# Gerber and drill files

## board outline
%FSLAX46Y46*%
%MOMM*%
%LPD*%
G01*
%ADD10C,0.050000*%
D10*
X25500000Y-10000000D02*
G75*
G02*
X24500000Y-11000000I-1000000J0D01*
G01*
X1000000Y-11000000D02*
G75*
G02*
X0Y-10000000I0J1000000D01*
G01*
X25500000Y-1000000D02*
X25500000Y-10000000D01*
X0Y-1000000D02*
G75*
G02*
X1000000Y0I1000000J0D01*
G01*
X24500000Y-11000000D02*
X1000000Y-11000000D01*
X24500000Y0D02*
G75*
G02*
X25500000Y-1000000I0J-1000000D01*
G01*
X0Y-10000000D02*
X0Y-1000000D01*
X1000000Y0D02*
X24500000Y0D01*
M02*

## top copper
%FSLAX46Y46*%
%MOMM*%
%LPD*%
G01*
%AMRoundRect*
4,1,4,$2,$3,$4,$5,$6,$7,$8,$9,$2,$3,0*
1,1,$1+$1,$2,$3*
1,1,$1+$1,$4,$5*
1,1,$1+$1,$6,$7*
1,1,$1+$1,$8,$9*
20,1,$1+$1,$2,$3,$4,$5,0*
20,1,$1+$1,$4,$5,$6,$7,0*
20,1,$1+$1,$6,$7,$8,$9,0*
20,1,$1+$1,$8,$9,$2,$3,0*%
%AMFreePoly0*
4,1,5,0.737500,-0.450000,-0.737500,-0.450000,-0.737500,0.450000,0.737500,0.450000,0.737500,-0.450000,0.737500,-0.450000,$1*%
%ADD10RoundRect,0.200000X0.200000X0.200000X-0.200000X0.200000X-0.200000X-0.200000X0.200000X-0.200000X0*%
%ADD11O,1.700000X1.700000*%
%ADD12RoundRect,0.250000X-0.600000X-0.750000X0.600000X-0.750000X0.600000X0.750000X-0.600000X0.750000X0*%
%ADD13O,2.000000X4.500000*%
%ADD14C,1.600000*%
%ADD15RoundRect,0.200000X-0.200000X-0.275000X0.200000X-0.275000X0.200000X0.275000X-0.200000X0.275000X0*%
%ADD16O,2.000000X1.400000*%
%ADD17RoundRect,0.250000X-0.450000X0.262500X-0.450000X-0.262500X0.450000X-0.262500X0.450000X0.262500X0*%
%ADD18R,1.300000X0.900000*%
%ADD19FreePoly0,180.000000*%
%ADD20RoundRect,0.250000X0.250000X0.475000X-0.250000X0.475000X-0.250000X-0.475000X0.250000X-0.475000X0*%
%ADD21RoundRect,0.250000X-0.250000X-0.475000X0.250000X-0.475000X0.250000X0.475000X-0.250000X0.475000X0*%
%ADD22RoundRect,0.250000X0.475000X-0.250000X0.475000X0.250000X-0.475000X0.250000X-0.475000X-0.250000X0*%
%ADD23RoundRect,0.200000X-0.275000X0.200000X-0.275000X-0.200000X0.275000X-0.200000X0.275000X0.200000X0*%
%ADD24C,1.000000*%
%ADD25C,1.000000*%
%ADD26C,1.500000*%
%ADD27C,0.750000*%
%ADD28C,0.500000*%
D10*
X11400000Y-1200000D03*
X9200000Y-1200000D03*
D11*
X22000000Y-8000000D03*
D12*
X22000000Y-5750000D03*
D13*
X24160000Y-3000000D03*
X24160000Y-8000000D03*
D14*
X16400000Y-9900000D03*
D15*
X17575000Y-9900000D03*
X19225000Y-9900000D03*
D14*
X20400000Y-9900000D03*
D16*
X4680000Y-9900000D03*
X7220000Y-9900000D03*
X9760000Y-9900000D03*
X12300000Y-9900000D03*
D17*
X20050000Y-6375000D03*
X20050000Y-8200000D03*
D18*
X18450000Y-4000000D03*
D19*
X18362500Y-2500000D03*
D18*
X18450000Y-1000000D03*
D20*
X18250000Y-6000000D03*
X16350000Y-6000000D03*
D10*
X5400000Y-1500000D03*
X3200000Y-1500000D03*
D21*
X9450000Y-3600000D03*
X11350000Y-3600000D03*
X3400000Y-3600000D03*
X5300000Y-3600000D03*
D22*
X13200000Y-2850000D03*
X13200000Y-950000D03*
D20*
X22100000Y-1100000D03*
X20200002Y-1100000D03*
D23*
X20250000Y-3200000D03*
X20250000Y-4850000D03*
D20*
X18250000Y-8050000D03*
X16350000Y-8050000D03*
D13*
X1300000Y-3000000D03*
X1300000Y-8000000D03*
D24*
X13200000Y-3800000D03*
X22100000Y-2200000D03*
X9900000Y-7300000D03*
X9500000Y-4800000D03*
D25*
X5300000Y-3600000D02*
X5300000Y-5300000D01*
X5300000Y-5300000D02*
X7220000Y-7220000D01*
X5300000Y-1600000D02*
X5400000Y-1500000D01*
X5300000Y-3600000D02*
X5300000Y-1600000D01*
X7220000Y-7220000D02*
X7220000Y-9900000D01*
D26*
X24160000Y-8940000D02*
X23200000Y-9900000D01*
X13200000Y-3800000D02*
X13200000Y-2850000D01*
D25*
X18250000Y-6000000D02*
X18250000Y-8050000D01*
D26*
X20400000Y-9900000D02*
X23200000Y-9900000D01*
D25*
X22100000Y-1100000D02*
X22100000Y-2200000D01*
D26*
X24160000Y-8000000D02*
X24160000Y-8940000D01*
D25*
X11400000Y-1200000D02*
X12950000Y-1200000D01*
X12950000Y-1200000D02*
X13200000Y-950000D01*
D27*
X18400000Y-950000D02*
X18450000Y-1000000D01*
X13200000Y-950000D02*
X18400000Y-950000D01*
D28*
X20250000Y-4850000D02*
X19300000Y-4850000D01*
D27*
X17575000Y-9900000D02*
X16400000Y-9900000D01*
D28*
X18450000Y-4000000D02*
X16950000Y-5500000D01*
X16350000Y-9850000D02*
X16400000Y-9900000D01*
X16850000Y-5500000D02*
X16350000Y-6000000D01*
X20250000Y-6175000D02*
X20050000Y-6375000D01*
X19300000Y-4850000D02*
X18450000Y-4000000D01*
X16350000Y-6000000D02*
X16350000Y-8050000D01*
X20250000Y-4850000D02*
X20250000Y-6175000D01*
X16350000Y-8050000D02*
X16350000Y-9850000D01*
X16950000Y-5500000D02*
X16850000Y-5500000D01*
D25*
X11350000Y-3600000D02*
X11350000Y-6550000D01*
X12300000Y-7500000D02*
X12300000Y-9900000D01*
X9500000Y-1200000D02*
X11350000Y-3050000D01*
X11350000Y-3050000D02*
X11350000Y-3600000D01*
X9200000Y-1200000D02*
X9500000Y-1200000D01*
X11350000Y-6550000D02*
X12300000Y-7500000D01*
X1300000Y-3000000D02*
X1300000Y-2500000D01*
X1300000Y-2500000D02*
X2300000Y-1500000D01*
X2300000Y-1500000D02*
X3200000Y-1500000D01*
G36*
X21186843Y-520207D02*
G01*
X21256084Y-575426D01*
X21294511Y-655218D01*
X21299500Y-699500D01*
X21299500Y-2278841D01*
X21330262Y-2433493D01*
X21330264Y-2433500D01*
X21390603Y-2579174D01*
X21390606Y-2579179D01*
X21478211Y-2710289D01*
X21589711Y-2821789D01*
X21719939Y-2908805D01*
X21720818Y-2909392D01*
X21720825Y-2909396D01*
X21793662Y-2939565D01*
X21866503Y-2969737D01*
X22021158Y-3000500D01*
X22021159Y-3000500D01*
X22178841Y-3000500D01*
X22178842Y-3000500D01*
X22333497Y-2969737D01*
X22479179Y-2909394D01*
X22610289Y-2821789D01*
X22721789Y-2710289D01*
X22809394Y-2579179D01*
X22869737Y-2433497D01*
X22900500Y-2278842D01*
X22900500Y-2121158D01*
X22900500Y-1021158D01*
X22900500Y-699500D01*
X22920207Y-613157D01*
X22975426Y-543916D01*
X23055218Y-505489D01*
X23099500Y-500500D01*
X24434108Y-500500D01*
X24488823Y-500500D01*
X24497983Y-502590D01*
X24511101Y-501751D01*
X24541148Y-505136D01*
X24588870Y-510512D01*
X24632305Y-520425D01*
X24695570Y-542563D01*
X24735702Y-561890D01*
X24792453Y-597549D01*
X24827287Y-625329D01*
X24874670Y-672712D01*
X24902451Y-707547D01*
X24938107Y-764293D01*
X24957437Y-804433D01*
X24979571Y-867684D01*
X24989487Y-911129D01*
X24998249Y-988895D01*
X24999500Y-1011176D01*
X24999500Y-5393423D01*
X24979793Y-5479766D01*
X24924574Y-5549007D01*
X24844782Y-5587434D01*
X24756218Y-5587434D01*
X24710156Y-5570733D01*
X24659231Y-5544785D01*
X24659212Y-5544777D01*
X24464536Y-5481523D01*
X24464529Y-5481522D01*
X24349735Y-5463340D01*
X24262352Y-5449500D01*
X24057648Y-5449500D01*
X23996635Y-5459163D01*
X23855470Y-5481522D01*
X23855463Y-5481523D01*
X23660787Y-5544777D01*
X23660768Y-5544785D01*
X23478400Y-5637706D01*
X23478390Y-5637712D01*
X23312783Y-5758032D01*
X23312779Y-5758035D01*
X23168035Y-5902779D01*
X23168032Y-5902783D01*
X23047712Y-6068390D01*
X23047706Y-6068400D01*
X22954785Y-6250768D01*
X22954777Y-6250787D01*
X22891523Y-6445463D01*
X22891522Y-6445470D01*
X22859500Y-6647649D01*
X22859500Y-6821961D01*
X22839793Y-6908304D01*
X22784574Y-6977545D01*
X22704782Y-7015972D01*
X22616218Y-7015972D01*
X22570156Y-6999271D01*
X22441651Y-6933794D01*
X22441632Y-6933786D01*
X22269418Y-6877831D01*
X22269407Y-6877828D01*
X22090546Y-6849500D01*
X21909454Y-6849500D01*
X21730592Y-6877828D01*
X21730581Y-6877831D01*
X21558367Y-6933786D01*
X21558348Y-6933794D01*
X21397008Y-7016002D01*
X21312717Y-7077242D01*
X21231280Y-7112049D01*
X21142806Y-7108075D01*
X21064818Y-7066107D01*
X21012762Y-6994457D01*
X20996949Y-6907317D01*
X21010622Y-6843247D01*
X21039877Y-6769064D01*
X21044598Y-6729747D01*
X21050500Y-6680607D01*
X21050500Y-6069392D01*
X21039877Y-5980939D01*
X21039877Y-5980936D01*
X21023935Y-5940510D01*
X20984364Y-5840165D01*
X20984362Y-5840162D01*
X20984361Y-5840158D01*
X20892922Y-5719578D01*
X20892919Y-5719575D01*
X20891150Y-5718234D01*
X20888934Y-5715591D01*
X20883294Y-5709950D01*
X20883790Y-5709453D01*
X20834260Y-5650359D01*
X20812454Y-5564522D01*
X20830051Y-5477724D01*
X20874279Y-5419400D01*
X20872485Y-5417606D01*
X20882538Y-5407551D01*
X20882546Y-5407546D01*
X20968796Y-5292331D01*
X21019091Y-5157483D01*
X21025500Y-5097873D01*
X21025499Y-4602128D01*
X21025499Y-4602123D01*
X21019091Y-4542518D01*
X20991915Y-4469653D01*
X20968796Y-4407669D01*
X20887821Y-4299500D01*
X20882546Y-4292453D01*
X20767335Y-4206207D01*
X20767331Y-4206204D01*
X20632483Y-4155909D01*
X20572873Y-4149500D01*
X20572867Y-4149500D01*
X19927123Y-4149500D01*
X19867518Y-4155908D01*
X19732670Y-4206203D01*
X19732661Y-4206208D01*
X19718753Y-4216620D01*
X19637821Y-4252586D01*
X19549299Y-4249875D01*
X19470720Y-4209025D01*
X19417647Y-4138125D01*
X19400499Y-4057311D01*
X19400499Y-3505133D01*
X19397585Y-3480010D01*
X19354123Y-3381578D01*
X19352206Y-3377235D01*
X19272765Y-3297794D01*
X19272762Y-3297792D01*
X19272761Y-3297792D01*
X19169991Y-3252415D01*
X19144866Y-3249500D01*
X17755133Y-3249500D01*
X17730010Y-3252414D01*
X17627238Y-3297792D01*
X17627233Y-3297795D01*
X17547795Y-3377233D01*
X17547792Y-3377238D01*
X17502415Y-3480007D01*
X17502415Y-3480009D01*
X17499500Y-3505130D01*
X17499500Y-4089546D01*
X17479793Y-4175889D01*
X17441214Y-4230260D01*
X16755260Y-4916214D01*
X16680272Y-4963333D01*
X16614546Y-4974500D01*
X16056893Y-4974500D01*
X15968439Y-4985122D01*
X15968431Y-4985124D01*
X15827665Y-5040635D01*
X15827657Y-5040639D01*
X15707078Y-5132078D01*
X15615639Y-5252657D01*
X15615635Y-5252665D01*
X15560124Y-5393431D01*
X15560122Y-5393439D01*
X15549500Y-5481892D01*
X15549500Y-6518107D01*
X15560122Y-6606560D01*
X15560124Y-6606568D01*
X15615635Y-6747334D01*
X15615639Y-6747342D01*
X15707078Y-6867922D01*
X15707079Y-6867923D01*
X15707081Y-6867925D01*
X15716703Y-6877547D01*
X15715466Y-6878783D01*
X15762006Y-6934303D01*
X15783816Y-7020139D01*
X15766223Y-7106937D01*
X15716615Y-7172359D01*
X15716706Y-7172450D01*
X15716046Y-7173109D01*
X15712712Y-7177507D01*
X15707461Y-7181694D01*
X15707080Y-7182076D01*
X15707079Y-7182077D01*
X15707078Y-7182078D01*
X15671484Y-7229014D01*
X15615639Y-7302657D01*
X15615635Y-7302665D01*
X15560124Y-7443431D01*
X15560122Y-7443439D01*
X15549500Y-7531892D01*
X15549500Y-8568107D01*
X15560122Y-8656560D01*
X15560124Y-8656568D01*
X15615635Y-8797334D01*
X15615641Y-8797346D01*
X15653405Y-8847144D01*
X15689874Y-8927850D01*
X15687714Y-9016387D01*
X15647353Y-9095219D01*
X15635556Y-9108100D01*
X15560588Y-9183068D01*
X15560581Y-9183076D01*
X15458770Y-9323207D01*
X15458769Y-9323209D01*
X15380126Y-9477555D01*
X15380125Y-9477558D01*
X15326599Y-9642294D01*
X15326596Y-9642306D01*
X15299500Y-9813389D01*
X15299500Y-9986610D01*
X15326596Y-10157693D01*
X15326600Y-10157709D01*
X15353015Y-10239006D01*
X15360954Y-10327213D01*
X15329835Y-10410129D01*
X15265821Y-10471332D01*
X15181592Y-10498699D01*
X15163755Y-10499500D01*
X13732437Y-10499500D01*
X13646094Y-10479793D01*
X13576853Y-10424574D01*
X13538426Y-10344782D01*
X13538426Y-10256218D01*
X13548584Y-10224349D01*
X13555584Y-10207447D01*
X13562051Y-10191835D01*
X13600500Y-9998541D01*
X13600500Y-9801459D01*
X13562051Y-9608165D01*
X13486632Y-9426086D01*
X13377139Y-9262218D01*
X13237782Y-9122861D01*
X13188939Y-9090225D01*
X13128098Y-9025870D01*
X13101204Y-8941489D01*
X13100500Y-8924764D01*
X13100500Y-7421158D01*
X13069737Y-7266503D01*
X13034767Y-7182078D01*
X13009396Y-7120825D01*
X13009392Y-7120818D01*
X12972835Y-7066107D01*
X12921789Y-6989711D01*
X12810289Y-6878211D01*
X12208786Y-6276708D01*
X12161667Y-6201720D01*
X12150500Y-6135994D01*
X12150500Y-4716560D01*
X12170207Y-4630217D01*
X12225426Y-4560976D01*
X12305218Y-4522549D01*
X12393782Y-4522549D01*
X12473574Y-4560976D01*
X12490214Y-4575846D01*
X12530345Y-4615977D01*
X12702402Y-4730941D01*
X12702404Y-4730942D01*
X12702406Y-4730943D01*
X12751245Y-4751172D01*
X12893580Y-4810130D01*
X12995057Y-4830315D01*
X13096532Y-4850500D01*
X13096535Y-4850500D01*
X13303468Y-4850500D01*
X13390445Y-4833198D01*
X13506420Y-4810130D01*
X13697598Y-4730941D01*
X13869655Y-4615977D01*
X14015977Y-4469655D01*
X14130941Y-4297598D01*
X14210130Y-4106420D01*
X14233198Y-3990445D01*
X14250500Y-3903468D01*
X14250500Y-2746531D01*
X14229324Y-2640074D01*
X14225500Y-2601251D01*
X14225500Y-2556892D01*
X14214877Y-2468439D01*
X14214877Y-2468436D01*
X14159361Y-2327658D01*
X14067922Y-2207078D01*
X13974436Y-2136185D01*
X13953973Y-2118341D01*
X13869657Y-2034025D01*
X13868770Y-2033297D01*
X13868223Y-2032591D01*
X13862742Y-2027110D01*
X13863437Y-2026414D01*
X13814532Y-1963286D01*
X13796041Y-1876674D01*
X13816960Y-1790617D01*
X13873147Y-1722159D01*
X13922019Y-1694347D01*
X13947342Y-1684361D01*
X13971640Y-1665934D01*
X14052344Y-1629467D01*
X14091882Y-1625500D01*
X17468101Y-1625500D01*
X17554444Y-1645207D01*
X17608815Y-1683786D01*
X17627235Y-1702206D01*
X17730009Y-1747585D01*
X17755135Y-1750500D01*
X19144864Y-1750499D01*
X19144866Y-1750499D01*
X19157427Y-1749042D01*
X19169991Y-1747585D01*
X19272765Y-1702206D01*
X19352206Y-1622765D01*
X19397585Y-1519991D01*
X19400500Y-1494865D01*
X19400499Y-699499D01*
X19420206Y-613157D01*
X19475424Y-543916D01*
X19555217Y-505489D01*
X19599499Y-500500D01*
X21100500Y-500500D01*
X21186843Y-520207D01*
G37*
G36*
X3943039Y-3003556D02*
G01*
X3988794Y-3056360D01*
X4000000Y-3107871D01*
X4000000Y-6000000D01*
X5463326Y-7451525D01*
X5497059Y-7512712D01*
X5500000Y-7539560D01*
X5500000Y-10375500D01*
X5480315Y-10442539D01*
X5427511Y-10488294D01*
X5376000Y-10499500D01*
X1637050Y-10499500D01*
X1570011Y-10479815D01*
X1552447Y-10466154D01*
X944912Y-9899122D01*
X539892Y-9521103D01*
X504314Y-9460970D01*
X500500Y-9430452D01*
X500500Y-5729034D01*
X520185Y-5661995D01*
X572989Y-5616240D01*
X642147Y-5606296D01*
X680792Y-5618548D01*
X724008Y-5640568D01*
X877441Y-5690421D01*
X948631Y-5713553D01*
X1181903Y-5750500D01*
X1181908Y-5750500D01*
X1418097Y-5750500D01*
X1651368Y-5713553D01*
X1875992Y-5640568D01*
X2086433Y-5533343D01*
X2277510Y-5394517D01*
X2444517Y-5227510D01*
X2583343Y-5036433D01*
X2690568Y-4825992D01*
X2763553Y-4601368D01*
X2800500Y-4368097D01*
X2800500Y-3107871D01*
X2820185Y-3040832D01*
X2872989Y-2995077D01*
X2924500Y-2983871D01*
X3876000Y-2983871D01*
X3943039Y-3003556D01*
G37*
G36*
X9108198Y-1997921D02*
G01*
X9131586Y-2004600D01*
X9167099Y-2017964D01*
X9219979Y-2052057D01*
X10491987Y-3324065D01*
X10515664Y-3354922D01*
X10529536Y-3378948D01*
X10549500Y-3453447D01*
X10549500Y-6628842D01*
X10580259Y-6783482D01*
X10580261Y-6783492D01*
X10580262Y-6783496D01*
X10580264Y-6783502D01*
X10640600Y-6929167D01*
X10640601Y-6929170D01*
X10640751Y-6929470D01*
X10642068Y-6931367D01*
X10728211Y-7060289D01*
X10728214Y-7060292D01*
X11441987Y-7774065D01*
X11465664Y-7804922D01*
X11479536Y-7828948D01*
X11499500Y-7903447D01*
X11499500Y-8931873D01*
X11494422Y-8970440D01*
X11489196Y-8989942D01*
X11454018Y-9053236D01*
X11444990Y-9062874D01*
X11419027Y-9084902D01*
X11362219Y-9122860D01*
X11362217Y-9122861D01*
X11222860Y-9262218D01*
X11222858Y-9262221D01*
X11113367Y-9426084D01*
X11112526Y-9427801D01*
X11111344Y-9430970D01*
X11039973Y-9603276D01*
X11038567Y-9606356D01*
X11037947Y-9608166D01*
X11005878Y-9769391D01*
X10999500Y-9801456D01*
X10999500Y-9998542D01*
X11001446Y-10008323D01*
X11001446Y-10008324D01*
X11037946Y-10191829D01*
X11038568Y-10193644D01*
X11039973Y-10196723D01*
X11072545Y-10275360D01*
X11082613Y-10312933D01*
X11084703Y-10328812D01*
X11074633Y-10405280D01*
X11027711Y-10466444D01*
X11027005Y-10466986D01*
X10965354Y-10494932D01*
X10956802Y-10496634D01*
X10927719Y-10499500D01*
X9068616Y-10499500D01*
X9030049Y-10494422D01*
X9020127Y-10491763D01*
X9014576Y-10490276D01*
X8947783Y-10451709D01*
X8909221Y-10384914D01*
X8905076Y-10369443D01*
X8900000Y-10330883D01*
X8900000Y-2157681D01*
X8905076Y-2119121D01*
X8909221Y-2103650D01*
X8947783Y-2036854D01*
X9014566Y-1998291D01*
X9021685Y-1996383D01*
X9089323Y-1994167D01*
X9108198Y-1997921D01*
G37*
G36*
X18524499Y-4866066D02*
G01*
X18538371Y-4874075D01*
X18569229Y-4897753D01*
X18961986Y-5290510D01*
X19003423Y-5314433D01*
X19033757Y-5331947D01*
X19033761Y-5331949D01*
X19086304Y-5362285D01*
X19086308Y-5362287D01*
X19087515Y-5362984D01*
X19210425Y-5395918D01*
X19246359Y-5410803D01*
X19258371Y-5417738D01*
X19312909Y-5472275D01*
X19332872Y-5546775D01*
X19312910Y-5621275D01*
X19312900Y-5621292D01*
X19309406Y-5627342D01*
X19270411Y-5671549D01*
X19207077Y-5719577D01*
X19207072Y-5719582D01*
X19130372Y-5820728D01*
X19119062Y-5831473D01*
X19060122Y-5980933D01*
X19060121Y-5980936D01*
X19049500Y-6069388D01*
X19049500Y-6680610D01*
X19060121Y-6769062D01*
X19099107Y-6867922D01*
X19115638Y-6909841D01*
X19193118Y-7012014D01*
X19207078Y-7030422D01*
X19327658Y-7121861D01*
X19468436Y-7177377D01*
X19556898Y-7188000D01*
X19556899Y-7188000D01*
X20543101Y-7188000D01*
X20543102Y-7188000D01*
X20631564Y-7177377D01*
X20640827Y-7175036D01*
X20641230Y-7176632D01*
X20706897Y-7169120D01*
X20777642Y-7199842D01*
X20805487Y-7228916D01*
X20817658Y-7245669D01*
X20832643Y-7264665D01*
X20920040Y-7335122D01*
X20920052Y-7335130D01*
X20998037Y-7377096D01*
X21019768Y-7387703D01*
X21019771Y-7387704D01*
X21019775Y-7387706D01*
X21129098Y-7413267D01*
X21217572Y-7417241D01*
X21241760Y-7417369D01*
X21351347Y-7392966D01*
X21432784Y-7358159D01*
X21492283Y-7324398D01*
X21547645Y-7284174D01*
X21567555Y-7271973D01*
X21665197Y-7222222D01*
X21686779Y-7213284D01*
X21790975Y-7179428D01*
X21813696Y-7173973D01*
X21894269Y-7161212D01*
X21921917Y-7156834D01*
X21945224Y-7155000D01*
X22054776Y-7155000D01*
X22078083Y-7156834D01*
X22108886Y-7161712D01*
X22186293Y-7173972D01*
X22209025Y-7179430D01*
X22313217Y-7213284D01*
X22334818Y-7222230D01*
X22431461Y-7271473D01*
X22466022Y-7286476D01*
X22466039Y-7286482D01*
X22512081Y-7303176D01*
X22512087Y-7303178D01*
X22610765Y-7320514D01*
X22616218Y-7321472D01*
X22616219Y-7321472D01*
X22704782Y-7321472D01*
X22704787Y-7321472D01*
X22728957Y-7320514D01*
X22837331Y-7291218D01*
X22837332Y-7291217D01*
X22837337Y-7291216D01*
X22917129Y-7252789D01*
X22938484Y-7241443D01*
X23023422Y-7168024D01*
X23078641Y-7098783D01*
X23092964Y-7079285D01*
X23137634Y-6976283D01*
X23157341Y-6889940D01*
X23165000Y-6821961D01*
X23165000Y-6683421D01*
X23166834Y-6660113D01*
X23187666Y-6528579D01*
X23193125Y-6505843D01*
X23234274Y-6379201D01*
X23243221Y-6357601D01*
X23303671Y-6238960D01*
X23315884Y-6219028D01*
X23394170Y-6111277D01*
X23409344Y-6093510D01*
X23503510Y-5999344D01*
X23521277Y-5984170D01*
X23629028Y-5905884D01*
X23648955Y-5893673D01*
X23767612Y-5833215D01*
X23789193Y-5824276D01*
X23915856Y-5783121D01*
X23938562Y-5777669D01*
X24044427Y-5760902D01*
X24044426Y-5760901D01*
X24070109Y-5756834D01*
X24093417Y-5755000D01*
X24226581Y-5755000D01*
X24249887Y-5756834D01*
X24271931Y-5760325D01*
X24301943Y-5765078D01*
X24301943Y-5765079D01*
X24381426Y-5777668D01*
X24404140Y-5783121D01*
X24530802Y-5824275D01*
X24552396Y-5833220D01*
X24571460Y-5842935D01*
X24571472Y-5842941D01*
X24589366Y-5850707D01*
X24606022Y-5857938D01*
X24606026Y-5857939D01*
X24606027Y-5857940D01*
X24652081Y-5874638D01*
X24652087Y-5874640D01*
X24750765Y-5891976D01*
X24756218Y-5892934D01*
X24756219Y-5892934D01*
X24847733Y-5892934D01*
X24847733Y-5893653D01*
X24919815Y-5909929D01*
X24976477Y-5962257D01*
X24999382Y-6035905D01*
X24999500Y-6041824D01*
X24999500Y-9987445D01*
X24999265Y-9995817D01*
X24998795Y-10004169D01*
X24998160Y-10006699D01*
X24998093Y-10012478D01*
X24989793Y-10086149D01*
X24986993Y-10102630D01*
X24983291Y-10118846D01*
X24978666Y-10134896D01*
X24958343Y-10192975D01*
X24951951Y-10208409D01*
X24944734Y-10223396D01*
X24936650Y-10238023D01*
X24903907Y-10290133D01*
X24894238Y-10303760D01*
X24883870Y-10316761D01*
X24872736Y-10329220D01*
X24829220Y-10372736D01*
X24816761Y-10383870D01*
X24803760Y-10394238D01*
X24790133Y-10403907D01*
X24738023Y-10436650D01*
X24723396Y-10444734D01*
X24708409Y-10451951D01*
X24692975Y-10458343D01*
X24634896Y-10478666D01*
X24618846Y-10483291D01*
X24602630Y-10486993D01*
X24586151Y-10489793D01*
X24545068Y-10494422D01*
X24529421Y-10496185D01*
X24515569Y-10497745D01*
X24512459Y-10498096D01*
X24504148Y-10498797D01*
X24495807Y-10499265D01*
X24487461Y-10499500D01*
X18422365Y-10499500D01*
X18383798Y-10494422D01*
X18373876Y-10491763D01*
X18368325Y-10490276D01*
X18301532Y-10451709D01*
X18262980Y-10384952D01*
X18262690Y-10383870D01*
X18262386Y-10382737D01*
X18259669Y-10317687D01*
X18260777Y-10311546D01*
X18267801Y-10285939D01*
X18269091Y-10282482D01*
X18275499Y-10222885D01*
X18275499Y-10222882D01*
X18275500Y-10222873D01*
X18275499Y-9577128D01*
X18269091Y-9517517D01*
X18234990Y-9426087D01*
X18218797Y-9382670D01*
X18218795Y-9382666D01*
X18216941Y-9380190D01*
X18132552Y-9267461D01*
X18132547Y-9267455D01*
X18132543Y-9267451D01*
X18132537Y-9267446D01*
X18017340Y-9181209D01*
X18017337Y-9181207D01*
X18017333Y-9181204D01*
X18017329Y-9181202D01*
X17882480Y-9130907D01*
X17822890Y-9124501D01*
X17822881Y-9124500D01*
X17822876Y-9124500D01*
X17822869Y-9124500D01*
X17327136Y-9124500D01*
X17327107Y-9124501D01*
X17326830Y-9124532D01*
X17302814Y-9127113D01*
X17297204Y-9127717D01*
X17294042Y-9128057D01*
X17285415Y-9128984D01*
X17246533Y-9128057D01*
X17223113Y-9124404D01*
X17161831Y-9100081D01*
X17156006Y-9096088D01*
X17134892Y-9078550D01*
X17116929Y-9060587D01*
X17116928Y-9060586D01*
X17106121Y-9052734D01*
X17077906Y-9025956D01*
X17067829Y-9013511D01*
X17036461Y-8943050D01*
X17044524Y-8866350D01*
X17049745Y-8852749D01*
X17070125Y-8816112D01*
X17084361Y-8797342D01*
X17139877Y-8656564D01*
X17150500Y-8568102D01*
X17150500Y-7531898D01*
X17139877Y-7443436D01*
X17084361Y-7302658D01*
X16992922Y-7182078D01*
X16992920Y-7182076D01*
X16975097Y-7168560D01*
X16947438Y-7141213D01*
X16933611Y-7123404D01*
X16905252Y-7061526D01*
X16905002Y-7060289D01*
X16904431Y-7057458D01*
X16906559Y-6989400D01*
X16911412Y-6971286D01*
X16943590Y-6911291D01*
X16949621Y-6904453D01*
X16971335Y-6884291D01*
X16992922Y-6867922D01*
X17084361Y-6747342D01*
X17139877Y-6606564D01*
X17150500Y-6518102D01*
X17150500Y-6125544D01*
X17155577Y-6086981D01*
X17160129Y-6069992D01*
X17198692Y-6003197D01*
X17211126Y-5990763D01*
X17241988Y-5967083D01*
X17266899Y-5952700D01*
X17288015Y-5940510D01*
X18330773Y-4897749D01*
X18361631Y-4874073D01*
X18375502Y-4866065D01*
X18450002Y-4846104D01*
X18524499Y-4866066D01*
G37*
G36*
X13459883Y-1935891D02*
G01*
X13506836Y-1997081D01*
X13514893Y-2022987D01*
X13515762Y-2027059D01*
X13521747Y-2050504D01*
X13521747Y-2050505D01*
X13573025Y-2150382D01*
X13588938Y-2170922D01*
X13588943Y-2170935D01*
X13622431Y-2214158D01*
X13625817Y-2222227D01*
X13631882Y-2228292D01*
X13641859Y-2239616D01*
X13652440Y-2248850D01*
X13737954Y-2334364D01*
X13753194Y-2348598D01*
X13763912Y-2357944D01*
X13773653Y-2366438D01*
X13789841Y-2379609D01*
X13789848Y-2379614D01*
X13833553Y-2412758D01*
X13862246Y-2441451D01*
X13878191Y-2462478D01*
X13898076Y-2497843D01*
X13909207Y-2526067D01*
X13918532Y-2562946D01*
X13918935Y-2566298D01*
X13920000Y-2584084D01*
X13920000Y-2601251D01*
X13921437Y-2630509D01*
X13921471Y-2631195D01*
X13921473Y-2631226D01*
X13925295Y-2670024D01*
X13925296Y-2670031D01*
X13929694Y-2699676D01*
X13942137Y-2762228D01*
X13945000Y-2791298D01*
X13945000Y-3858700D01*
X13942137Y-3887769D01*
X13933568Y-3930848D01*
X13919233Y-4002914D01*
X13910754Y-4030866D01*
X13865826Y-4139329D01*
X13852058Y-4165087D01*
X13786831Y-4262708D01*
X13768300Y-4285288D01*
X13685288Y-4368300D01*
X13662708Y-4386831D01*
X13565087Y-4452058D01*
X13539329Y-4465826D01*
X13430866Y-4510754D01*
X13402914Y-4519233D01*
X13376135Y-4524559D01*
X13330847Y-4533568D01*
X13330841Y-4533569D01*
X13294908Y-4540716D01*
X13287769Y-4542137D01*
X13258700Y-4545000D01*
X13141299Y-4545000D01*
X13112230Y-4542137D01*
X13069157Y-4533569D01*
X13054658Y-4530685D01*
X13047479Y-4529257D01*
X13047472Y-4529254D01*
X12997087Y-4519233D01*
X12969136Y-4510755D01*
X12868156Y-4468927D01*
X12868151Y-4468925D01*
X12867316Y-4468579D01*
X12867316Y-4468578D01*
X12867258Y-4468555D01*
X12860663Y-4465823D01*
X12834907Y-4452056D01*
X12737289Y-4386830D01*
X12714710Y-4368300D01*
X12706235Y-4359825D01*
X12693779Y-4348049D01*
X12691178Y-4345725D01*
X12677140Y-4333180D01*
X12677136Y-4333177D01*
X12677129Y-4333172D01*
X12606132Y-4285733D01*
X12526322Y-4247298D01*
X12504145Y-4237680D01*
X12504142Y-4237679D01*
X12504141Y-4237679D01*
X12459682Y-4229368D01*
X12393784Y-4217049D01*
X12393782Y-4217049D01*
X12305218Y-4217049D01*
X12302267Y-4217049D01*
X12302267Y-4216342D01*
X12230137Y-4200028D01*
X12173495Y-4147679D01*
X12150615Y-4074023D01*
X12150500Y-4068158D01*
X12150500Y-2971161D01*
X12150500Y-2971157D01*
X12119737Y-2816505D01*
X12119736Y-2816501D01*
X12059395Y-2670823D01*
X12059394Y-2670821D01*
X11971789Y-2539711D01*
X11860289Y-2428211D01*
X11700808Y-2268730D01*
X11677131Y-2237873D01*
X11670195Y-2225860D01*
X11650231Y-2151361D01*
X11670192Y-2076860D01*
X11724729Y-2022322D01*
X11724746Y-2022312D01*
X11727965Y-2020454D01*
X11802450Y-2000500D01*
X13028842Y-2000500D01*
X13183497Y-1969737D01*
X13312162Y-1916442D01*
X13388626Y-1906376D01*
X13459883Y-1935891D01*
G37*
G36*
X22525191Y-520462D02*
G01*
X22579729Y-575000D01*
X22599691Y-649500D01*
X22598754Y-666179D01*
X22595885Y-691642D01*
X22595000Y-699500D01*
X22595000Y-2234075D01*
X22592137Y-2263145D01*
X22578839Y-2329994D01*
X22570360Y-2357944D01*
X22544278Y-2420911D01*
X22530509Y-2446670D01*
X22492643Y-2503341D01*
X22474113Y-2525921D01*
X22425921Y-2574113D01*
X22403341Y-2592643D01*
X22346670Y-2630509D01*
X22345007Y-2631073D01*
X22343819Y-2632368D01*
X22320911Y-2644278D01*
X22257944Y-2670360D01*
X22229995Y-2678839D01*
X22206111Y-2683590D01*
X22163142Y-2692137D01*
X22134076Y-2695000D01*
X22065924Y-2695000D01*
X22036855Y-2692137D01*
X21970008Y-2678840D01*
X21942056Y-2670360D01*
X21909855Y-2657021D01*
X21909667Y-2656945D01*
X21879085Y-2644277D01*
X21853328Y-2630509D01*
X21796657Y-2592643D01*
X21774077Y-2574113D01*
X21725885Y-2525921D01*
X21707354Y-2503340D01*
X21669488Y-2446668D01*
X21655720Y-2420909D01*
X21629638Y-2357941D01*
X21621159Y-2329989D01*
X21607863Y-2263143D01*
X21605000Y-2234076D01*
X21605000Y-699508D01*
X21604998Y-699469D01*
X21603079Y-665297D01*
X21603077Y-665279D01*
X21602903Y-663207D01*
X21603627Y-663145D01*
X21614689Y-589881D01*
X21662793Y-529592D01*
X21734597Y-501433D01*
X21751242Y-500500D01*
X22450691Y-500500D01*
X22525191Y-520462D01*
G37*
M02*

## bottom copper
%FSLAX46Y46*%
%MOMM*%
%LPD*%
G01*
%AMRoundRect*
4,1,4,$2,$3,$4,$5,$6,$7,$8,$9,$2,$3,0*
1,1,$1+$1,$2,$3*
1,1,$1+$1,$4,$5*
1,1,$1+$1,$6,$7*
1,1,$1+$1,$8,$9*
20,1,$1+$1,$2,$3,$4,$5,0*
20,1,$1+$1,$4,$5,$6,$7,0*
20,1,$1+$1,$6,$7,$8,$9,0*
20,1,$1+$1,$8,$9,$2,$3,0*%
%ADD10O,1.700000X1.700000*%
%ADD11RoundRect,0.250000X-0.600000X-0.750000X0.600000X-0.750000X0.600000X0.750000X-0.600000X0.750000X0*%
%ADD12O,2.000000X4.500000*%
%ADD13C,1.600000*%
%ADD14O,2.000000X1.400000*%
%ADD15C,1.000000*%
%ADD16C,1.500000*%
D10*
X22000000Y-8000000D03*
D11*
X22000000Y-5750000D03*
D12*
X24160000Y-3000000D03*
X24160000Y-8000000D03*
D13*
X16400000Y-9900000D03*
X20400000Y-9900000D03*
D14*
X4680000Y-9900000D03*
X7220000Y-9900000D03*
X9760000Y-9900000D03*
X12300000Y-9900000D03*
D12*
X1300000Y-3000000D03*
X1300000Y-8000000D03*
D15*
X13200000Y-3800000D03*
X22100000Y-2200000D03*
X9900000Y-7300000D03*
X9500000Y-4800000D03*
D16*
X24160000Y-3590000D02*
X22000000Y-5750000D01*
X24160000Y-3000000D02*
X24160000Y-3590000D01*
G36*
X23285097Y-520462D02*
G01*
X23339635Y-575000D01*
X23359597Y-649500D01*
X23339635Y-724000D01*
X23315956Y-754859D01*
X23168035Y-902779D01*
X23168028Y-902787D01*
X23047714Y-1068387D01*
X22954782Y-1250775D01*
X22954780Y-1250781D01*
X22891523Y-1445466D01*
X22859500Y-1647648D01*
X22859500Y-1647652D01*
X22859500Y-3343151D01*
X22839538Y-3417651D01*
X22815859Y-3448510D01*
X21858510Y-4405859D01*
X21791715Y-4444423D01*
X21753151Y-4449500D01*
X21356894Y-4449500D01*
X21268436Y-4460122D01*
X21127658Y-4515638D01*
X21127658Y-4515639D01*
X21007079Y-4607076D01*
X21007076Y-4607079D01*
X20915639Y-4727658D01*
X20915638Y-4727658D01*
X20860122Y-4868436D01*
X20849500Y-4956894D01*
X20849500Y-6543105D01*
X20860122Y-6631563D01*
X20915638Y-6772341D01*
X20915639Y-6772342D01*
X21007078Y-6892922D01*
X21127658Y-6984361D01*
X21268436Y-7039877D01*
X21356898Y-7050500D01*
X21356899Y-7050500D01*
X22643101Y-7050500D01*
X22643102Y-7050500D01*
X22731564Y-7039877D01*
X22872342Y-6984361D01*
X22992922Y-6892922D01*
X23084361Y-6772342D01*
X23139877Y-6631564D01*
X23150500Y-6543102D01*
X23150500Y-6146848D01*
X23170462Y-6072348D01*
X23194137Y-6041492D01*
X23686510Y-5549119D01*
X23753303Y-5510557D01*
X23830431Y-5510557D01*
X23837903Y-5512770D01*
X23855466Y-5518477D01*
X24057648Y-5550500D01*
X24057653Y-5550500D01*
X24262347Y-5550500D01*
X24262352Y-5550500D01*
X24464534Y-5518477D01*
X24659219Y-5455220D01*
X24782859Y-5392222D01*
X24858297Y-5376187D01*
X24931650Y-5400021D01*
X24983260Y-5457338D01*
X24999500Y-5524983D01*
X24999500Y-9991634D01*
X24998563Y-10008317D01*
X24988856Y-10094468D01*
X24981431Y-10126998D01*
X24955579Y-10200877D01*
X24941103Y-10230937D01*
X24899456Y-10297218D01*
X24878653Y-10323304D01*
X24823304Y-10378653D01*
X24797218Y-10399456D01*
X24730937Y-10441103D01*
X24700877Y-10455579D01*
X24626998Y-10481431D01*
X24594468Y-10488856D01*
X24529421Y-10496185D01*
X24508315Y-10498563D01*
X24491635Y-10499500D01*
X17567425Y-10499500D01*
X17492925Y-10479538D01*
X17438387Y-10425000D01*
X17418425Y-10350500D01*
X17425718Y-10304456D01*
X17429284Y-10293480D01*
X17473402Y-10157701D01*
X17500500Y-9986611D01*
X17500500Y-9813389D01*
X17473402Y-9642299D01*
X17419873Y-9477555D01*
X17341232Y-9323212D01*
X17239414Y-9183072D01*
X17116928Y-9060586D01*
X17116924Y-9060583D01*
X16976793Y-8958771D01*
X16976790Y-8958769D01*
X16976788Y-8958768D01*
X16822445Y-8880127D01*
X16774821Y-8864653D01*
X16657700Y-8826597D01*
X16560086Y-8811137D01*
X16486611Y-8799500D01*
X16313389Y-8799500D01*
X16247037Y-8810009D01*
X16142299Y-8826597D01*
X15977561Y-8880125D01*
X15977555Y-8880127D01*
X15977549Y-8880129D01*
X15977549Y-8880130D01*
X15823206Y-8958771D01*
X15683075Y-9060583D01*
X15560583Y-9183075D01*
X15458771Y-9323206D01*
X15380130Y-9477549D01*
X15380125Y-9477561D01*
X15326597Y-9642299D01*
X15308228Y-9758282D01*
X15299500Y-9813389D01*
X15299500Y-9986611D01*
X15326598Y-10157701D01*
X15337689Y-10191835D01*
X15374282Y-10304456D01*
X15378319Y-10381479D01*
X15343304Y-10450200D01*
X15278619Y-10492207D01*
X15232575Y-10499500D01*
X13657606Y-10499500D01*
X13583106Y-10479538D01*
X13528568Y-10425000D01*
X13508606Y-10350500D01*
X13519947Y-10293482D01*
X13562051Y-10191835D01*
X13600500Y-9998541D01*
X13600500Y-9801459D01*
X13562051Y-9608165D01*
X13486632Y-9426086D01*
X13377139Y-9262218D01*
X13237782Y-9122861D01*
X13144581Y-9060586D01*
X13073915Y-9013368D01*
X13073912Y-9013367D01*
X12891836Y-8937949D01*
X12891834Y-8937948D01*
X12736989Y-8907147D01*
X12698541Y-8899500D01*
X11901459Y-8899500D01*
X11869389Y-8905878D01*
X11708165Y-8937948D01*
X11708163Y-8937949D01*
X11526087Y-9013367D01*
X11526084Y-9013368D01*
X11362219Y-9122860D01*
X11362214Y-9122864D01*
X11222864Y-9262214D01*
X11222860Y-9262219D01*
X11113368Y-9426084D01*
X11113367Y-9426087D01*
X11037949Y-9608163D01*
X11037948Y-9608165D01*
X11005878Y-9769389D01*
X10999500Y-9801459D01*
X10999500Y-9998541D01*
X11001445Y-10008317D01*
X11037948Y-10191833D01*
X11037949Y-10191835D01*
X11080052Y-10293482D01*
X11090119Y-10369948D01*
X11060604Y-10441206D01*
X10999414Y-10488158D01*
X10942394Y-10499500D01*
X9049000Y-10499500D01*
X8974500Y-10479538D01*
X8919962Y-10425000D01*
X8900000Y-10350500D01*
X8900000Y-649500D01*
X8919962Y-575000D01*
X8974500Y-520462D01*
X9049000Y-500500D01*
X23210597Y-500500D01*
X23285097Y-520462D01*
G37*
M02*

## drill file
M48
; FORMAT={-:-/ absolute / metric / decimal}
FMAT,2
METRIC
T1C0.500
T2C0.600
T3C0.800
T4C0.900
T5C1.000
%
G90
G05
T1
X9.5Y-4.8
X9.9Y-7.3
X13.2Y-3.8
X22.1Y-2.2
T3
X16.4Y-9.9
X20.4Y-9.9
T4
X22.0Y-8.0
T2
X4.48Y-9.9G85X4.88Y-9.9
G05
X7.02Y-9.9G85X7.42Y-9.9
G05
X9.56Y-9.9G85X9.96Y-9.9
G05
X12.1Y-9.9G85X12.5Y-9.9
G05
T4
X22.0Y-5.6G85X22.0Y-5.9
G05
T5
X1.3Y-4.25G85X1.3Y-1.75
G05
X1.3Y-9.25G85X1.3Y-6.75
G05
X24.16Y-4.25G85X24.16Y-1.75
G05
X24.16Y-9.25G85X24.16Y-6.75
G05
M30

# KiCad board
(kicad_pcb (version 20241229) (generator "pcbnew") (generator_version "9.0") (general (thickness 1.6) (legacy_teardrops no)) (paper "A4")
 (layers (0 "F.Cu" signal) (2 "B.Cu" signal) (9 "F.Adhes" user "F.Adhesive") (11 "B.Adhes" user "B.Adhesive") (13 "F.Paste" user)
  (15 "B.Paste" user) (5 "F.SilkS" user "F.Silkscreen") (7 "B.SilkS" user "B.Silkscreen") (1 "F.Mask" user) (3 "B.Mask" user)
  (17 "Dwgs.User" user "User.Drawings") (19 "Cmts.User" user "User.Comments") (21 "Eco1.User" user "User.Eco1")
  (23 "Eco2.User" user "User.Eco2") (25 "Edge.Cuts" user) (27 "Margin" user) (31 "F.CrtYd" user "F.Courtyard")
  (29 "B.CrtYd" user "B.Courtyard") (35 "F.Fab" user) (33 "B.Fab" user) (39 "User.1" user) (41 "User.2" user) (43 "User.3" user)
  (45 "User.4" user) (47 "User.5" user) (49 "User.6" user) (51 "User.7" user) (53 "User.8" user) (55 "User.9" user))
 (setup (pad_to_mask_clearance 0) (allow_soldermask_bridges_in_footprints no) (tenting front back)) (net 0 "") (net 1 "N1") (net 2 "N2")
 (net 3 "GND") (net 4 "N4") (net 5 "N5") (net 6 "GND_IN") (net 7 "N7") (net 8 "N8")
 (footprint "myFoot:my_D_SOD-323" (layer "F.Cu") (at 10.3 1.2 180)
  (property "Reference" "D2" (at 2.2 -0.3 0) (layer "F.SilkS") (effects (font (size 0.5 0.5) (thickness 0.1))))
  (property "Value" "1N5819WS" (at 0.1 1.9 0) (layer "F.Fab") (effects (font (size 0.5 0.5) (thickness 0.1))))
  (pad "1" smd roundrect (at -1.1 0 180) (size 0.8 0.8) (layers "F.Cu" "F.Mask" "F.Paste") (roundrect_rratio 0.25) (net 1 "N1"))
  (pad "2" smd roundrect (at 1.1 0 180) (size 0.8 0.8) (layers "F.Cu" "F.Mask" "F.Paste") (roundrect_rratio 0.25) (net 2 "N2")))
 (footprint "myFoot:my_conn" (layer "F.Cu") (at 22 6.95)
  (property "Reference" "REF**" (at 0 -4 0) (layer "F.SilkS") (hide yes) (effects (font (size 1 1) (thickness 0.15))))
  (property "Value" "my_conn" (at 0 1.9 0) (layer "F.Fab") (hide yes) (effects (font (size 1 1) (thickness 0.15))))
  (pad "1" thru_hole oval (at 0 1.05) (size 1.7 1.7) (drill oval 0.9) (layers "*.Cu" "*.Mask") (remove_unused_layers no) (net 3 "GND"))
  (pad "2" thru_hole roundrect (at 0 -1.2) (size 1.7 2) (drill oval 0.9 1.2) (layers "*.Cu" "*.Mask") (remove_unused_layers no)
   (roundrect_rratio 0.1470588235) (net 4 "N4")))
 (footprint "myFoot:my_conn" (layer "F.Cu") (at 24.16 5.5 180)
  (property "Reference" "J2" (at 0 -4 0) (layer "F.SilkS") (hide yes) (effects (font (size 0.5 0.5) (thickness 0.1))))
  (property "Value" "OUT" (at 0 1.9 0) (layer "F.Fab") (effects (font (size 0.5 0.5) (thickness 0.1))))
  (pad "1" thru_hole oval (at 0 2.5 180) (size 2 4.5) (drill oval 1 3.5) (layers "*.Cu" "*.Mask") (remove_unused_layers no) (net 4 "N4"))
  (pad "2" thru_hole oval (at 0 -2.5 180) (size 2 4.5) (drill oval 1 3.5) (layers "*.Cu" "*.Mask") (remove_unused_layers no) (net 3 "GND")))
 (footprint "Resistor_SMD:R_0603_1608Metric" (layer "F.Cu") (at 18.4 9.9)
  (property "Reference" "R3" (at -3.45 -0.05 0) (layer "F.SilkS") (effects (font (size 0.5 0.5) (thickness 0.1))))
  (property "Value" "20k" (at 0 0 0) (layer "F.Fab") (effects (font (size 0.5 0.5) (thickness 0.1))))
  (pad "1" thru_hole circle (at -2 0) (size 1.6 1.6) (drill 0.8) (layers "*.Cu" "*.Mask") (remove_unused_layers no) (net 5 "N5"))
  (pad "1" smd roundrect (at -0.825 0) (size 0.8 0.95) (layers "F.Cu" "F.Mask" "F.Paste") (roundrect_rratio 0.25) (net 5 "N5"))
  (pad "2" smd roundrect (at 0.825 0) (size 0.8 0.95) (layers "F.Cu" "F.Mask" "F.Paste") (roundrect_rratio 0.25) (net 3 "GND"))
  (pad "2" thru_hole circle (at 2 0) (size 1.6 1.6) (drill 0.8) (layers "*.Cu" "*.Mask") (remove_unused_layers no) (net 3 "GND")))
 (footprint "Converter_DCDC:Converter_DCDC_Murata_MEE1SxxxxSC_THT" (layer "F.Cu") (at 8.49 9.9 90)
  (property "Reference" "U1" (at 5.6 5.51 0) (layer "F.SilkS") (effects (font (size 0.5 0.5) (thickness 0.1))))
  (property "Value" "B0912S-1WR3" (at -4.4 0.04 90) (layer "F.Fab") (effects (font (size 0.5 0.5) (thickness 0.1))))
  (pad "1" thru_hole oval (at 0 -3.81 90) (size 1.4 2) (drill oval 0.6 1) (layers "*.Cu" "*.Mask") (remove_unused_layers no)
   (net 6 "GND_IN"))
  (pad "2" thru_hole oval (at 0 -1.27 90) (size 1.4 2) (drill oval 0.6 1) (layers "*.Cu" "*.Mask") (remove_unused_layers no) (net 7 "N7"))
  (pad "3" thru_hole oval (at 0 1.27 90) (size 1.4 2) (drill oval 0.6 1) (layers "*.Cu" "*.Mask") (remove_unused_layers no) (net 3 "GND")
   (zone_connect 2))
  (pad "4" thru_hole oval (at 0 3.81 90) (size 1.4 2) (drill oval 0.6 1) (layers "*.Cu" "*.Mask") (remove_unused_layers no) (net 2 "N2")))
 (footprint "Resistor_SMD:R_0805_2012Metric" (layer "F.Cu") (at 20.05 7.2875 -90)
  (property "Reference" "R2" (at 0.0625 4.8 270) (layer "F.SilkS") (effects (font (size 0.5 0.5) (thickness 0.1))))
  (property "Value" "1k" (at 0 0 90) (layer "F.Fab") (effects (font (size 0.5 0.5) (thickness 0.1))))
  (pad "1" smd roundrect (at -0.9125 0 270) (size 1.025 1.4) (layers "F.Cu" "F.Mask" "F.Paste") (roundrect_rratio 0.243902) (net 5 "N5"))
  (pad "2" smd roundrect (at 0.9125 0 270) (size 1.025 1.4) (layers "F.Cu" "F.Mask" "F.Paste") (roundrect_rratio 0.243902) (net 3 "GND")))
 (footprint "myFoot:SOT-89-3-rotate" (layer "F.Cu") (at 17 2.5 180)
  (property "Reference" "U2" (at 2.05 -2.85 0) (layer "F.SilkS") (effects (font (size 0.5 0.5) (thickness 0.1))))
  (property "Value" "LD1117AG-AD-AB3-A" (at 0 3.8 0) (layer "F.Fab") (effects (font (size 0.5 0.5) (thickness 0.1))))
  (pad "1" smd rect (at -1.45 -1.5 180) (size 1.3 0.9) (layers "F.Cu" "F.Mask" "F.Paste") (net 5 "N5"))
  (pad "2" smd custom (at -1.3625 0 180) (size 1.475 0.9) (layers "F.Cu" "F.Mask" "F.Paste") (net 4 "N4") (zone_connect 2)
   (options (clearance outline) (anchor rect)) (primitives))
  (pad "3" smd rect (at -1.45 1.5 180) (size 1.3 0.9) (layers "F.Cu" "F.Mask" "F.Paste") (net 1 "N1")))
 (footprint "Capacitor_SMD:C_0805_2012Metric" (layer "F.Cu") (at 17.3 6 180)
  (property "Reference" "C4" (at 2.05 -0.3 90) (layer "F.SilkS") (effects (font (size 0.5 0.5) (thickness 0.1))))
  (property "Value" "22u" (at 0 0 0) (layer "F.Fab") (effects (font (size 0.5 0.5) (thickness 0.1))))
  (pad "1" smd roundrect (at -0.95 0 180) (size 1 1.45) (layers "F.Cu" "F.Mask" "F.Paste") (roundrect_rratio 0.25) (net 3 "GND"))
  (pad "2" smd roundrect (at 0.95 0 180) (size 1 1.45) (layers "F.Cu" "F.Mask" "F.Paste") (roundrect_rratio 0.25) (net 5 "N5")))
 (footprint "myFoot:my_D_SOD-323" (layer "F.Cu") (at 4.3 1.5 180)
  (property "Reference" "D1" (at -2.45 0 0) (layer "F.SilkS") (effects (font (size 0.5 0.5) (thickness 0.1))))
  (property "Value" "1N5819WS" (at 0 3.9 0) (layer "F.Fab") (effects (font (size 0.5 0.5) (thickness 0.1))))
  (pad "1" smd roundrect (at -1.1 0 180) (size 0.8 0.8) (layers "F.Cu" "F.Mask" "F.Paste") (roundrect_rratio 0.25) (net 7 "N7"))
  (pad "2" smd roundrect (at 1.1 0 180) (size 0.8 0.8) (layers "F.Cu" "F.Mask" "F.Paste") (roundrect_rratio 0.25) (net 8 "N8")))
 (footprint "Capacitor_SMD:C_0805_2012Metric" (layer "F.Cu") (at 10.4 3.6)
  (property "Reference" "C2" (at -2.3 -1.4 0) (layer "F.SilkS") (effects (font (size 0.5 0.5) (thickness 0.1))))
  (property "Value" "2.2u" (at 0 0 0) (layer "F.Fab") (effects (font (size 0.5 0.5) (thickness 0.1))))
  (pad "1" smd roundrect (at -0.95 0) (size 1 1.45) (layers "F.Cu" "F.Mask" "F.Paste") (roundrect_rratio 0.25) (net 3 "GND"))
  (pad "2" smd roundrect (at 0.95 0) (size 1 1.45) (layers "F.Cu" "F.Mask" "F.Paste") (roundrect_rratio 0.25) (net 2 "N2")))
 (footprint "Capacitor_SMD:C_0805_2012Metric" (layer "F.Cu") (at 4.35 3.6)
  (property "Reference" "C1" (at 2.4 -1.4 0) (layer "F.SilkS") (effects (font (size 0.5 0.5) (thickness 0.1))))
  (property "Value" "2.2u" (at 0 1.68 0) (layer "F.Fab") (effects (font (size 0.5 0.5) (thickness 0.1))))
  (pad "1" smd roundrect (at -0.95 0) (size 1 1.45) (layers "F.Cu" "F.Mask" "F.Paste") (roundrect_rratio 0.25) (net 6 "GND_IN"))
  (pad "2" smd roundrect (at 0.95 0) (size 1 1.45) (layers "F.Cu" "F.Mask" "F.Paste") (roundrect_rratio 0.25) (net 7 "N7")))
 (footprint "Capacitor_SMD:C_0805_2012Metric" (layer "F.Cu") (at 13.2 1.9 90)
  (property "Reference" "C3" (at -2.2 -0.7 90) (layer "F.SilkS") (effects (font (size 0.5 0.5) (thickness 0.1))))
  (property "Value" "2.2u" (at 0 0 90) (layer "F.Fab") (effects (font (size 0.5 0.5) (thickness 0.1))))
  (pad "1" smd roundrect (at -0.95 0 90) (size 1 1.45) (layers "F.Cu" "F.Mask" "F.Paste") (roundrect_rratio 0.25) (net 3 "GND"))
  (pad "2" smd roundrect (at 0.95 0 90) (size 1 1.45) (layers "F.Cu" "F.Mask" "F.Paste") (roundrect_rratio 0.25) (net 1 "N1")))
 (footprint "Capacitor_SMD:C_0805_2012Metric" (layer "F.Cu") (at 21.150001 1.1 180)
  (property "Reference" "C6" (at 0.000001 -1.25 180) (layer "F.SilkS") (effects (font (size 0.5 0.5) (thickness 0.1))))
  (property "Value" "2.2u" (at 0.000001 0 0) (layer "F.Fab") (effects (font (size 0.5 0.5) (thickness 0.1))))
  (pad "1" smd roundrect (at -0.949999 0 180) (size 1 1.45) (layers "F.Cu" "F.Mask" "F.Paste") (roundrect_rratio 0.25) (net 3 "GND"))
  (pad "2" smd roundrect (at 0.949999 0 180) (size 1 1.45) (layers "F.Cu" "F.Mask" "F.Paste") (roundrect_rratio 0.25) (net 4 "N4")))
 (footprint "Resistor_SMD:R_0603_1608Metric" (layer "F.Cu") (at 20.25 4.025 -90)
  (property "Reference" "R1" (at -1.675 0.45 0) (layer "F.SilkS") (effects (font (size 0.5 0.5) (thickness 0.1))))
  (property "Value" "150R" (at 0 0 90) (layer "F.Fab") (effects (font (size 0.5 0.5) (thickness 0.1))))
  (pad "1" smd roundrect (at -0.825 0 270) (size 0.8 0.95) (layers "F.Cu" "F.Mask" "F.Paste") (roundrect_rratio 0.25) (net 4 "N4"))
  (pad "2" smd roundrect (at 0.825 0 270) (size 0.8 0.95) (layers "F.Cu" "F.Mask" "F.Paste") (roundrect_rratio 0.25) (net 5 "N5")))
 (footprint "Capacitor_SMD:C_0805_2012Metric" (layer "F.Cu") (at 17.3 8.05 180)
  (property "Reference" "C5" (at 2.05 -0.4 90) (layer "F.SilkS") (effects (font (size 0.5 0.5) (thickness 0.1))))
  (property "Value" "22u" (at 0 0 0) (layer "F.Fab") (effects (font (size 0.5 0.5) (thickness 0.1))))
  (pad "1" smd roundrect (at -0.95 0 180) (size 1 1.45) (layers "F.Cu" "F.Mask" "F.Paste") (roundrect_rratio 0.25) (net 3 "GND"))
  (pad "2" smd roundrect (at 0.95 0 180) (size 1 1.45) (layers "F.Cu" "F.Mask" "F.Paste") (roundrect_rratio 0.25) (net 5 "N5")))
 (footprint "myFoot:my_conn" (layer "F.Cu") (at 1.3 5.5 180)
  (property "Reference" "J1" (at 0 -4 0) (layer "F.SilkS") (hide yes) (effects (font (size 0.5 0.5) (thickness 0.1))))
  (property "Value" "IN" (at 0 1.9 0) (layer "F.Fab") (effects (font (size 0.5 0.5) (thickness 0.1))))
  (pad "1" thru_hole oval (at 0 2.5 180) (size 2 4.5) (drill oval 1 3.5) (layers "*.Cu" "*.Mask") (remove_unused_layers no) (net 8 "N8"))
  (pad "2" thru_hole oval (at 0 -2.5 180) (size 2 4.5) (drill oval 1 3.5) (layers "*.Cu" "*.Mask") (remove_unused_layers no)
   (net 6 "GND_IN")))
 (gr_arc (start 25.5 10) (mid 25.207107 10.707107) (end 24.5 11) (stroke (width 0.05) (type default)) (layer "Edge.Cuts"))
 (gr_arc (start 1 11) (mid 0.292893 10.707107) (end 0 10) (stroke (width 0.05) (type default)) (layer "Edge.Cuts"))
 (gr_line (start 25.5 1) (end 25.5 10) (stroke (width 0.05) (type default)) (layer "Edge.Cuts"))
 (gr_arc (start 0 1) (mid 0.292893 0.292893) (end 1 0) (stroke (width 0.05) (type default)) (layer "Edge.Cuts"))
 (gr_line (start 24.5 11) (end 1 11) (stroke (width 0.05) (type default)) (layer "Edge.Cuts"))
 (gr_arc (start 24.5 0) (mid 25.207107 0.292893) (end 25.5 1) (stroke (width 0.05) (type default)) (layer "Edge.Cuts"))
 (gr_line (start 0 10) (end 0 1) (stroke (width 0.05) (type default)) (layer "Edge.Cuts"))
 (gr_line (start 1 0) (end 24.5 0) (stroke (width 0.05) (type default)) (layer "Edge.Cuts"))
 (segment (start 5.3 3.6) (end 5.3 5.3) (width 1) (layer "F.Cu") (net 7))
 (segment (start 5.3 5.3) (end 7.22 7.22) (width 1) (layer "F.Cu") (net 7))
 (segment (start 5.3 1.6) (end 5.4 1.5) (width 1) (layer "F.Cu") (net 7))
 (segment (start 5.3 3.6) (end 5.3 1.6) (width 1) (layer "F.Cu") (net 7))
 (segment (start 7.22 7.22) (end 7.22 9.9) (width 1) (layer "F.Cu") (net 7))
 (segment (start 24.16 8.94) (end 23.2 9.9) (width 1.5) (layer "F.Cu") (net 3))
 (segment (start 13.2 3.8) (end 13.2 2.85) (width 1.5) (layer "F.Cu") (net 3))
 (segment (start 18.25 6) (end 18.25 8.05) (width 1) (layer "F.Cu") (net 3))
 (segment (start 20.4 9.9) (end 23.2 9.9) (width 1.5) (layer "F.Cu") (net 3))
 (segment (start 22.1 1.1) (end 22.1 2.2) (width 1) (layer "F.Cu") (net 3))
 (segment (start 24.16 8) (end 24.16 8.94) (width 1.5) (layer "F.Cu") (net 3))
 (via (at 13.2 3.8) (size 1) (drill 0.5) (layers "F.Cu" "B.Cu") (free yes) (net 3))
 (via (at 22.1 2.2) (size 1) (drill 0.5) (layers "F.Cu" "B.Cu") (free yes) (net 3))
 (via (at 9.9 7.3) (size 1) (drill 0.5) (layers "F.Cu" "B.Cu") (free yes) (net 3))
 (via (at 9.5 4.8) (size 1) (drill 0.5) (layers "F.Cu" "B.Cu") (free yes) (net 3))
 (segment (start 11.4 1.2) (end 12.95 1.2) (width 1) (layer "F.Cu") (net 1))
 (segment (start 12.95 1.2) (end 13.2 0.95) (width 1) (layer "F.Cu") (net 1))
 (segment (start 18.4 0.95) (end 18.45 1) (width 0.75) (layer "F.Cu") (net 1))
 (segment (start 13.2 0.95) (end 18.4 0.95) (width 0.75) (layer "F.Cu") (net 1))
 (segment (start 20.25 4.85) (end 19.3 4.85) (width 0.5) (layer "F.Cu") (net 5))
 (segment (start 17.575 9.9) (end 16.4 9.9) (width 0.75) (layer "F.Cu") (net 5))
 (segment (start 18.45 4) (end 16.95 5.5) (width 0.5) (layer "F.Cu") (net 5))
 (segment (start 16.35 9.85) (end 16.4 9.9) (width 0.5) (layer "F.Cu") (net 5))
 (segment (start 16.85 5.5) (end 16.35 6) (width 0.5) (layer "F.Cu") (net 5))
 (segment (start 20.25 6.175) (end 20.05 6.375) (width 0.5) (layer "F.Cu") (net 5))
 (segment (start 19.3 4.85) (end 18.45 4) (width 0.5) (layer "F.Cu") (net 5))
 (segment (start 16.35 6) (end 16.35 8.05) (width 0.5) (layer "F.Cu") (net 5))
 (segment (start 20.25 4.85) (end 20.25 6.175) (width 0.5) (layer "F.Cu") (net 5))
 (segment (start 16.35 8.05) (end 16.35 9.85) (width 0.5) (layer "F.Cu") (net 5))
 (segment (start 16.95 5.5) (end 16.85 5.5) (width 0.5) (layer "F.Cu") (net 5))
 (segment (start 11.35 3.6) (end 11.35 6.55) (width 1) (layer "F.Cu") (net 2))
 (segment (start 12.3 7.5) (end 12.3 9.9) (width 1) (layer "F.Cu") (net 2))
 (segment (start 9.5 1.2) (end 11.35 3.05) (width 1) (layer "F.Cu") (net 2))
 (segment (start 11.35 3.05) (end 11.35 3.6) (width 1) (layer "F.Cu") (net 2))
 (segment (start 9.2 1.2) (end 9.5 1.2) (width 1) (layer "F.Cu") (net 2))
 (segment (start 11.35 6.55) (end 12.3 7.5) (width 1) (layer "F.Cu") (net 2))
 (segment (start 1.3 3) (end 1.3 2.5) (width 1) (layer "F.Cu") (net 8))
 (segment (start 1.3 2.5) (end 2.3 1.5) (width 1) (layer "F.Cu") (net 8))
 (segment (start 2.3 1.5) (end 3.2 1.5) (width 1) (layer "F.Cu") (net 8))
 (segment (start 24.16 3.59) (end 22 5.75) (width 1.5) (layer "B.Cu") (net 4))
 (segment (start 24.16 3) (end 24.16 3.59) (width 1.5) (layer "B.Cu") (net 4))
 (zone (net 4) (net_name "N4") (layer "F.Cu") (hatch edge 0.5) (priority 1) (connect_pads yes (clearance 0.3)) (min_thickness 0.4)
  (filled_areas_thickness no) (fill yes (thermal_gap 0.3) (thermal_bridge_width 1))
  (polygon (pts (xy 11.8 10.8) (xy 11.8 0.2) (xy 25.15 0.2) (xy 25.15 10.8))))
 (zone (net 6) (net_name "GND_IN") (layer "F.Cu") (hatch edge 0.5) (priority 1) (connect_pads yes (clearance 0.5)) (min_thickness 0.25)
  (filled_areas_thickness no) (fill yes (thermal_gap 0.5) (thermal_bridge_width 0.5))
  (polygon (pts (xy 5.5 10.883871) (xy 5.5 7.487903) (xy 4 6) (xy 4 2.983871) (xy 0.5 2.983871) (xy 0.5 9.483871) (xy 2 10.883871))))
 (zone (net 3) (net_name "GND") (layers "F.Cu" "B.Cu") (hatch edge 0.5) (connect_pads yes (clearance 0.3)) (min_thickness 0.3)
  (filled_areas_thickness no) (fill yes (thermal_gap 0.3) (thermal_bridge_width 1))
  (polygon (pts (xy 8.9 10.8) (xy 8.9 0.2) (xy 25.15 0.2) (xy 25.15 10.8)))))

